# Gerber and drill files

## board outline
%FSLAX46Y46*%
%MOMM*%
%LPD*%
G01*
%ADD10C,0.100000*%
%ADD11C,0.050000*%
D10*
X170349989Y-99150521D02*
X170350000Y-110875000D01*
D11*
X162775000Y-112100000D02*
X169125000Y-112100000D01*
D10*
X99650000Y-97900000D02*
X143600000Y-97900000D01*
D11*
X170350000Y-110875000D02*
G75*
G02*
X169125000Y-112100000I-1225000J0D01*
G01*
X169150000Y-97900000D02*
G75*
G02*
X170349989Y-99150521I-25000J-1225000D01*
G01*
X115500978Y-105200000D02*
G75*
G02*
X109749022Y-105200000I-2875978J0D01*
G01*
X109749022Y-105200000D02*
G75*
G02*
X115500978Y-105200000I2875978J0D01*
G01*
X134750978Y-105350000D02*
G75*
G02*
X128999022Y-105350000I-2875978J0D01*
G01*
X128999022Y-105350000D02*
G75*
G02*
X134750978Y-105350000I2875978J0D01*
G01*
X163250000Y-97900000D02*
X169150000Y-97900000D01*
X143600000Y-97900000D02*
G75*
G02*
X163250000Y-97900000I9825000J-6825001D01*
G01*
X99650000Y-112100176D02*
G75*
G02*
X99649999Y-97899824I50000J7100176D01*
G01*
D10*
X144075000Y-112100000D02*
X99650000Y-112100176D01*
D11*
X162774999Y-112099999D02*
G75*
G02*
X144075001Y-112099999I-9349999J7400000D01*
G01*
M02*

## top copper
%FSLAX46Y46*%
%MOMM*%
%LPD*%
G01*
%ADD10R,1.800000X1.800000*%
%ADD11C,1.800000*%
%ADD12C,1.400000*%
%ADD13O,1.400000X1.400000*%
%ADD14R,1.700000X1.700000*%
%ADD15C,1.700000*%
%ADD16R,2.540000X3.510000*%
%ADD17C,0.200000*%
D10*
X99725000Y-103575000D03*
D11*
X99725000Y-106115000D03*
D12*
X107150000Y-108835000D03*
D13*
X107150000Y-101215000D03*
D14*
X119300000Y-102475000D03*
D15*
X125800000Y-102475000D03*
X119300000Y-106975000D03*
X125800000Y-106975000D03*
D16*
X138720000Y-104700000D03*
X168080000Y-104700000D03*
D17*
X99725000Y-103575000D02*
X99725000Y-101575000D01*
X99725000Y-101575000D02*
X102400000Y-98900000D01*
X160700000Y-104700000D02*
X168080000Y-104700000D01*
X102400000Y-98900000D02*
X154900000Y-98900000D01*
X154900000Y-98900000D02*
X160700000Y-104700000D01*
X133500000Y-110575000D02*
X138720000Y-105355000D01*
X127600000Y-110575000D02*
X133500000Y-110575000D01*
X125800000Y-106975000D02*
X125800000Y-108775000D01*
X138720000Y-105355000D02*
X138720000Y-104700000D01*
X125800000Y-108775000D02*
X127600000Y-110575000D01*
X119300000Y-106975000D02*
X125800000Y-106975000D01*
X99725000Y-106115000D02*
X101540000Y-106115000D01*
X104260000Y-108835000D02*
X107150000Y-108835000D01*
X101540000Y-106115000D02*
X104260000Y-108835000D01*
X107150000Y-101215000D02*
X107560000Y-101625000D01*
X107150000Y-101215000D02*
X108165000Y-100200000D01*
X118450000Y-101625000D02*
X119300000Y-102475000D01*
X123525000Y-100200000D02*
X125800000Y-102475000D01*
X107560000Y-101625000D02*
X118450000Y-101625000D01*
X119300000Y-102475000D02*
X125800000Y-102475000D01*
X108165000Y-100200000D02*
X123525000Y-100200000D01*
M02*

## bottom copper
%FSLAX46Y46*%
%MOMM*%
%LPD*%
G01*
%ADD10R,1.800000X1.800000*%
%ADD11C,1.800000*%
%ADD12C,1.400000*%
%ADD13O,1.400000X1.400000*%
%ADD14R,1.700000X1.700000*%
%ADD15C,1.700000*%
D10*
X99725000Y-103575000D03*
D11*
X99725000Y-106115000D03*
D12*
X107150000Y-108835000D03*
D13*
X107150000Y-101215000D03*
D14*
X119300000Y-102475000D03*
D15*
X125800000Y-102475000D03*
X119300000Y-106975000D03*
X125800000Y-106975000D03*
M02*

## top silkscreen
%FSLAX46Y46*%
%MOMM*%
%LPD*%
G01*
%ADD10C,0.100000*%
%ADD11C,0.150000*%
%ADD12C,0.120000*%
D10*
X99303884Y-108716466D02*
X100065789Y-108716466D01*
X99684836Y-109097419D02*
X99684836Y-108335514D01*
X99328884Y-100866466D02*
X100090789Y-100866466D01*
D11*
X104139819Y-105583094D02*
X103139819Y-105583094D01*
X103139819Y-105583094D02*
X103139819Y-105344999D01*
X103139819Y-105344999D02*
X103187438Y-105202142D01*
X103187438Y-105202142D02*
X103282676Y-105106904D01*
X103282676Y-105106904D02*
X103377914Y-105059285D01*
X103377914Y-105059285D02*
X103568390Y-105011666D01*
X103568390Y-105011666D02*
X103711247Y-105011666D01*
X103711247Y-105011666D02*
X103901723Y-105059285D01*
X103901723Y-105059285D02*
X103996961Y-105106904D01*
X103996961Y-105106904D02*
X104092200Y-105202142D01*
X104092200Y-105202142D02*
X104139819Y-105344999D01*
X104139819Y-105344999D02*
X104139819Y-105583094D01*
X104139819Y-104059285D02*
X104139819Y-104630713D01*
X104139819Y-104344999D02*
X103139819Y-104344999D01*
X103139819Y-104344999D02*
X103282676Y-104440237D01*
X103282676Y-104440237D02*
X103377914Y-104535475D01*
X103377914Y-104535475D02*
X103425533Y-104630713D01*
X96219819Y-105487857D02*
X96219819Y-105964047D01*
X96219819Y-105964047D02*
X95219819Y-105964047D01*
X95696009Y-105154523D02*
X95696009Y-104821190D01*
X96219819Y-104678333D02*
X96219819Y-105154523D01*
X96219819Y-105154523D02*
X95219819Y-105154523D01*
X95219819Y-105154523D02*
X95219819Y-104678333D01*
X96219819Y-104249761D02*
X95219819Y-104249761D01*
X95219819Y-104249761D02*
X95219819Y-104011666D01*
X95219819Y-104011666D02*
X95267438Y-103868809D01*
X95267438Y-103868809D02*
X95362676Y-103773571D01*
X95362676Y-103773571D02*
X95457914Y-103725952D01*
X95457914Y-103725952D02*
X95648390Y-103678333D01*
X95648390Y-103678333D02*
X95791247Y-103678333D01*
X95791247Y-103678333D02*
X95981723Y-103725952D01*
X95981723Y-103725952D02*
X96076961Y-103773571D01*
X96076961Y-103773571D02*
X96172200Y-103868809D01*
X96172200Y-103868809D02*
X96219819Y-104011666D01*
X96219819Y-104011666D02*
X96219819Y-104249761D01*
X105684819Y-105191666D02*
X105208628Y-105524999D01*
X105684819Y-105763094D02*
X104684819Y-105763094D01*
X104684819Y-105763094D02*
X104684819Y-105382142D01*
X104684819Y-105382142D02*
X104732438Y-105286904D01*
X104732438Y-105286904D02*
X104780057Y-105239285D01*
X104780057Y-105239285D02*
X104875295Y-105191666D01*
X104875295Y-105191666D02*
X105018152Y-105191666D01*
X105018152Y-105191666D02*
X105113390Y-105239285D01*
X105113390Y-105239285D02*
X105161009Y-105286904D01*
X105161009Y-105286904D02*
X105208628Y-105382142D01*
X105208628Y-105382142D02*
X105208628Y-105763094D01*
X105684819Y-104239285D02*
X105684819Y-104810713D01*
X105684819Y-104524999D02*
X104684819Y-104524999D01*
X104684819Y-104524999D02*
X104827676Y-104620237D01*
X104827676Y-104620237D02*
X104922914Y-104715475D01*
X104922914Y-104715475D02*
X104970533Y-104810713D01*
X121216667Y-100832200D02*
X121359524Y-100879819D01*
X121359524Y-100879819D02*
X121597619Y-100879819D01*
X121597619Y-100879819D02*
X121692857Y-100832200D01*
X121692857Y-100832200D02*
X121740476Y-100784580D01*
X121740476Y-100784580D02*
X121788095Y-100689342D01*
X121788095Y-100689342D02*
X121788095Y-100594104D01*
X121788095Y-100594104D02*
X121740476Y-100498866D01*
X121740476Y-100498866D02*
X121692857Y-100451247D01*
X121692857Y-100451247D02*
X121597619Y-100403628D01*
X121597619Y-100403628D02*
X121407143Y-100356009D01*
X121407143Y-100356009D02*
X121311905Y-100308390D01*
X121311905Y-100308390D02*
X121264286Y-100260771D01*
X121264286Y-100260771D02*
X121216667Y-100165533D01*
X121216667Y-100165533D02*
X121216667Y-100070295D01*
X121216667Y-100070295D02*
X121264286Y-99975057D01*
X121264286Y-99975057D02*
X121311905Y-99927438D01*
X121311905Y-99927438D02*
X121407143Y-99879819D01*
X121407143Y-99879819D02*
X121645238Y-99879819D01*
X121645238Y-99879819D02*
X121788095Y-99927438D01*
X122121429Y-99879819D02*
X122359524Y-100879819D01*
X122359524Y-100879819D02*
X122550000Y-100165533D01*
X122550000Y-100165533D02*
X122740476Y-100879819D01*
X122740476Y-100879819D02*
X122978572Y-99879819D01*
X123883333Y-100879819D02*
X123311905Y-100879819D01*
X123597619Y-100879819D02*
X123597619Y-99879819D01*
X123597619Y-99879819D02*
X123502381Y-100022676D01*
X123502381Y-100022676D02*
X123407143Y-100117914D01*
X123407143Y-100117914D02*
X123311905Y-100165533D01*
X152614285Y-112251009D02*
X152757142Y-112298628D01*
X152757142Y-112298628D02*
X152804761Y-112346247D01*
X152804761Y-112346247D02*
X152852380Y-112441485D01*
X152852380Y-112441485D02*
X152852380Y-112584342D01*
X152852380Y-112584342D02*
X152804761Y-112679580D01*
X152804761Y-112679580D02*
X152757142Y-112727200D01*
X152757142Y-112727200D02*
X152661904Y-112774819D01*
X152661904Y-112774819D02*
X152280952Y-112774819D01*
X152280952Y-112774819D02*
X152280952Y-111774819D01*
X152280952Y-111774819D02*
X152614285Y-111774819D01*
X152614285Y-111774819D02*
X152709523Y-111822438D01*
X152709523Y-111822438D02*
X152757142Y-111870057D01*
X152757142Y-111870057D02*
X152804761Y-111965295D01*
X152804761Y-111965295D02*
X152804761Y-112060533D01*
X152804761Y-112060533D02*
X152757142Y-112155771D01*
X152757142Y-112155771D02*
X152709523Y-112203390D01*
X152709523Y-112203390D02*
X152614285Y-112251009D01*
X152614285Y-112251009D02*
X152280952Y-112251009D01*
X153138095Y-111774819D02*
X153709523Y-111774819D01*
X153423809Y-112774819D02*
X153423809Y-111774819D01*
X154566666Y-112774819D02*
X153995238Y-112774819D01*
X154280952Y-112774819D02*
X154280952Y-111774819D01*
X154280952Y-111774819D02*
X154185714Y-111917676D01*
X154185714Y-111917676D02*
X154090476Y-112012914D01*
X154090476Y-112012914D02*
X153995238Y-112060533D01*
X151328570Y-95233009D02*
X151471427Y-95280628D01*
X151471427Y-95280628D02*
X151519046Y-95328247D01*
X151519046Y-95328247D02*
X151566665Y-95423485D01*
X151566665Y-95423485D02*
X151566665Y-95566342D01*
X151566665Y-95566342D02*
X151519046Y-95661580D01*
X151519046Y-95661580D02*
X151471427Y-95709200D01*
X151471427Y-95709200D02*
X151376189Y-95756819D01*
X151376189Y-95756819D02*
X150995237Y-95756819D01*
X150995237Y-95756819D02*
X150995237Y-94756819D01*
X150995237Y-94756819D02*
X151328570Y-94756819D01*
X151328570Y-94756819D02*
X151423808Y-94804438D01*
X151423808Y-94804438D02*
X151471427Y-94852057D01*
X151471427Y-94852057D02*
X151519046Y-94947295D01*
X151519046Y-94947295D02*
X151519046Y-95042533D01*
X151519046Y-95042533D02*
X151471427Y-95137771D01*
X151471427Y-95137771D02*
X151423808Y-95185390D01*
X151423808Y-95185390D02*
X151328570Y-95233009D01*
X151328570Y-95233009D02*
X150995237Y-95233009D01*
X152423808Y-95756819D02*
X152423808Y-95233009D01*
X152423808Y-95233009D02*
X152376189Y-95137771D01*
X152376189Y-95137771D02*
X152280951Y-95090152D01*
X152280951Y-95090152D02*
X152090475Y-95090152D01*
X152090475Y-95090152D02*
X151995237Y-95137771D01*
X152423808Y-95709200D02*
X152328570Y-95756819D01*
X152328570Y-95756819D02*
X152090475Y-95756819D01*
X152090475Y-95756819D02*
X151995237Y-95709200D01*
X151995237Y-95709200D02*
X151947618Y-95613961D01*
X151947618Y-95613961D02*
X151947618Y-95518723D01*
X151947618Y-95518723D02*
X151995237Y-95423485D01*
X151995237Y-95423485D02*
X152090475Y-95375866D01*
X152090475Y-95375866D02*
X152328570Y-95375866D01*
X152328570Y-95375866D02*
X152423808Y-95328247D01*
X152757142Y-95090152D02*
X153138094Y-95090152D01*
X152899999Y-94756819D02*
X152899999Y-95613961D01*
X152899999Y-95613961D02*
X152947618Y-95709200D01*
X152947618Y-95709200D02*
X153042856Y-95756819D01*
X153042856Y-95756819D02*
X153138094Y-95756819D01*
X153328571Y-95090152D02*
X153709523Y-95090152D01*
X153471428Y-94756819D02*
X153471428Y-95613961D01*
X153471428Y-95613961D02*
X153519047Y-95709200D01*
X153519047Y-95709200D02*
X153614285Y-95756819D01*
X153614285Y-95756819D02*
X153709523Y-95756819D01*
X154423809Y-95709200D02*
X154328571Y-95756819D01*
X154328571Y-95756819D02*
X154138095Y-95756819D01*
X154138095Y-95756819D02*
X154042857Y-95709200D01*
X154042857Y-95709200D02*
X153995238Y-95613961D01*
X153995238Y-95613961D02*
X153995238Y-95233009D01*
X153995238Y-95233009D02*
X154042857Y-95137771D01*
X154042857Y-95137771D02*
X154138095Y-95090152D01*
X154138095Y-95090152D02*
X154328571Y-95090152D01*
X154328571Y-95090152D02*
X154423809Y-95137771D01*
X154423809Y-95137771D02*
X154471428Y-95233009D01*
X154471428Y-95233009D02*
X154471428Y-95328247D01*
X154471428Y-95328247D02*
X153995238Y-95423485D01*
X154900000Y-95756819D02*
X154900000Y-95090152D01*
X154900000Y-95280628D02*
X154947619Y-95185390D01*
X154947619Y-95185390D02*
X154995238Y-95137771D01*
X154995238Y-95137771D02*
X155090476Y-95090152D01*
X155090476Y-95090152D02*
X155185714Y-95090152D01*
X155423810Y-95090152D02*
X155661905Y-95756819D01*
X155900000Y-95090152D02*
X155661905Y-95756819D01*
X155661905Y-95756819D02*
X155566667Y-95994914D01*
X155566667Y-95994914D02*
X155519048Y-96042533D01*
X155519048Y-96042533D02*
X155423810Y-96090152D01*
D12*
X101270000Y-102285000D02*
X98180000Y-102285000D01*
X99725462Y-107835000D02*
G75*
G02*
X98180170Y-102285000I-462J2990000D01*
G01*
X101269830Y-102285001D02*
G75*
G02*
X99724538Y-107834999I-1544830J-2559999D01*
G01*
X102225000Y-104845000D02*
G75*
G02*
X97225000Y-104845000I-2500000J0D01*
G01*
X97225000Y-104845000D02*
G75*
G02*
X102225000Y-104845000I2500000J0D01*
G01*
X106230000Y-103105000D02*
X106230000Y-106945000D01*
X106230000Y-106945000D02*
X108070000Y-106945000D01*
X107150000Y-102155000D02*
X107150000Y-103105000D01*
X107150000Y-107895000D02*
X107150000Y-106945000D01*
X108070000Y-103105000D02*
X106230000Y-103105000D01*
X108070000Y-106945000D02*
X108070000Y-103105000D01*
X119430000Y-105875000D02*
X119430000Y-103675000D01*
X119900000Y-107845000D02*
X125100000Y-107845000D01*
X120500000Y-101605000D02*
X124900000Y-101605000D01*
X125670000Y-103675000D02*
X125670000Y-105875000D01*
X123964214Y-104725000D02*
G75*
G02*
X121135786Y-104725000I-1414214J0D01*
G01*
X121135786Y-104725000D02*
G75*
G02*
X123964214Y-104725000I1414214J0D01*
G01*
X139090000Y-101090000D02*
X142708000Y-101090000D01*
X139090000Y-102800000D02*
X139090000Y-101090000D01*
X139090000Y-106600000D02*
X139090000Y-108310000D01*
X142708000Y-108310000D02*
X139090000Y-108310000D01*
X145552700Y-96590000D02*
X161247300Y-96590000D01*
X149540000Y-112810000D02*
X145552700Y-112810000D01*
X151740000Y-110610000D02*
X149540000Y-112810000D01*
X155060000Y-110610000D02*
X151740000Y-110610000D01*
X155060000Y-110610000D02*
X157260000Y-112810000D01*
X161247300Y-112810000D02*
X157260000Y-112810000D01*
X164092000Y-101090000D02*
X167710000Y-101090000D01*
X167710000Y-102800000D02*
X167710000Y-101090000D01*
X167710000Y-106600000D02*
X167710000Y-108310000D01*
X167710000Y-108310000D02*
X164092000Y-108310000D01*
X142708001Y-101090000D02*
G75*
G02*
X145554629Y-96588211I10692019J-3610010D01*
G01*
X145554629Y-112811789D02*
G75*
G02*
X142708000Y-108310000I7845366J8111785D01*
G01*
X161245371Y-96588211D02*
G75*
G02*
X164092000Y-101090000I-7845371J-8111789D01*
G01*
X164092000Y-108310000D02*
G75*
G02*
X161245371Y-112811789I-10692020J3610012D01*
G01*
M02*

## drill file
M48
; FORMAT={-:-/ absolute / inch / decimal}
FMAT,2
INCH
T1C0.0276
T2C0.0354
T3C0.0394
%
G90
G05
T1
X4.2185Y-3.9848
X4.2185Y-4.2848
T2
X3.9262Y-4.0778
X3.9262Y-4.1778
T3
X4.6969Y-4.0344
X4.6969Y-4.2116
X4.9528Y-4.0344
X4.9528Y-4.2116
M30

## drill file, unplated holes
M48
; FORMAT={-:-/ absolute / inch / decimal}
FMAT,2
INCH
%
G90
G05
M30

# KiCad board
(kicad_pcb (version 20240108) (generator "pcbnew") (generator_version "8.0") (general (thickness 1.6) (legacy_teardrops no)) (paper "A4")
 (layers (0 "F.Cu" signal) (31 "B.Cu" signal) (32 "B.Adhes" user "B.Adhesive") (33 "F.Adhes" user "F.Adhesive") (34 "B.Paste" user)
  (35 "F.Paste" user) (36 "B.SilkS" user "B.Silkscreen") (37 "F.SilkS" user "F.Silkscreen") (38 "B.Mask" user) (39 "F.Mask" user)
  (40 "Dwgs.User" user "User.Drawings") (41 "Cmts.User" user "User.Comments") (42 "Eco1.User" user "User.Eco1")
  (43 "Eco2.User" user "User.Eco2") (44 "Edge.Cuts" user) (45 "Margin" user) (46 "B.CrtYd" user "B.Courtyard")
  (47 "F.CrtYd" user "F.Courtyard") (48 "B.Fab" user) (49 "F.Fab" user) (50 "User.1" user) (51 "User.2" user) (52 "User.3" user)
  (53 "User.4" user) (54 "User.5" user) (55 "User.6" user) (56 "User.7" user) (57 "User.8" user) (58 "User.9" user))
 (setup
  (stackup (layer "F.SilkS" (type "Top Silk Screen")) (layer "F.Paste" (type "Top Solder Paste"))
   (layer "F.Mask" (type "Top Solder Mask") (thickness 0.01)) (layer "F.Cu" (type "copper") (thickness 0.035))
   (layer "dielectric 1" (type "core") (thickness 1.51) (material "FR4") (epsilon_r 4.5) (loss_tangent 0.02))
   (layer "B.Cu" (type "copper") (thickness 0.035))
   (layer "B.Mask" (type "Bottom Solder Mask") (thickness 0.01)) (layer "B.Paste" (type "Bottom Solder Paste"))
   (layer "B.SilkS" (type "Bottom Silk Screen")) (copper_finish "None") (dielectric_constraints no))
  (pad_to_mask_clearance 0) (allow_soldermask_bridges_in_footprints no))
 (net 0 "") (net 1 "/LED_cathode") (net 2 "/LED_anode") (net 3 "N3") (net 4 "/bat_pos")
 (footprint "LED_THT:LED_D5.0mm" (layer "F.Cu") (at 99.725 103.575 -90)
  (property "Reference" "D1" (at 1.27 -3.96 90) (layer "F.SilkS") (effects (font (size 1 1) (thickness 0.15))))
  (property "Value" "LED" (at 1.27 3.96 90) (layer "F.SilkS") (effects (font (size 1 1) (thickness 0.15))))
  (fp_line (start -1.29 -1.545) (end -1.29 1.545) (stroke (width 0.12) (type solid)) (layer "F.SilkS"))
  (fp_arc (start 4.26 -0.000462) (mid 2.072002 2.880433) (end -1.29 1.54483) (stroke (width 0.12) (type solid)) (layer "F.SilkS"))
  (fp_arc (start -1.29 -1.54483) (mid 2.072002 -2.880433) (end 4.26 0.000462) (stroke (width 0.12) (type solid)) (layer "F.SilkS"))
  (fp_circle (center 1.27 0) (end 3.77 0) (stroke (width 0.12) (type solid)) (fill none) (layer "F.SilkS"))
  (pad "1" thru_hole rect (at 0 0 270) (size 1.8 1.8) (drill 0.9) (layers "*.Cu" "*.Mask") (remove_unused_layers no) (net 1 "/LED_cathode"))
  (pad "2" thru_hole circle (at 2.54 0 270) (size 1.8 1.8) (drill 0.9) (layers "*.Cu" "*.Mask") (remove_unused_layers no)
   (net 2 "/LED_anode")))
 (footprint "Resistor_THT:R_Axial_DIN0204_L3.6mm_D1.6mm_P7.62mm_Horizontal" (layer "F.Cu") (at 107.15 108.835 90)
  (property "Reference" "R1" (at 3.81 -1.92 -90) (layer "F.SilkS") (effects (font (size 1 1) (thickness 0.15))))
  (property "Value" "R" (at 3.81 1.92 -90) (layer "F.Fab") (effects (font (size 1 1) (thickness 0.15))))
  (fp_line (start 5.73 -0.92) (end 1.89 -0.92) (stroke (width 0.12) (type solid)) (layer "F.SilkS"))
  (fp_line (start 1.89 -0.92) (end 1.89 0.92) (stroke (width 0.12) (type solid)) (layer "F.SilkS"))
  (fp_line (start 6.68 0) (end 5.73 0) (stroke (width 0.12) (type solid)) (layer "F.SilkS"))
  (fp_line (start 0.94 0) (end 1.89 0) (stroke (width 0.12) (type solid)) (layer "F.SilkS"))
  (fp_line (start 5.73 0.92) (end 5.73 -0.92) (stroke (width 0.12) (type solid)) (layer "F.SilkS"))
  (fp_line (start 1.89 0.92) (end 5.73 0.92) (stroke (width 0.12) (type solid)) (layer "F.SilkS"))
  (pad "1" thru_hole circle (at 0 0 90) (size 1.4 1.4) (drill 0.7) (layers "*.Cu" "*.Mask") (remove_unused_layers no) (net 2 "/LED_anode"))
  (pad "2" thru_hole oval (at 7.62 0 90) (size 1.4 1.4) (drill 0.7) (layers "*.Cu" "*.Mask") (remove_unused_layers no) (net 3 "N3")))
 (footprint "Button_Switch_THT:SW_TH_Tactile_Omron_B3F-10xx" (layer "F.Cu") (at 119.3 102.475)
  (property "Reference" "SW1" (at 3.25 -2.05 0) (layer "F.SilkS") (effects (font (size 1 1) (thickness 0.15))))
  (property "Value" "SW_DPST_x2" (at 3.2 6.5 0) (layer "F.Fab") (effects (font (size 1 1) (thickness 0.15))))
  (fp_line (start 0.13 3.4) (end 0.13 1.2) (stroke (width 0.12) (type solid)) (layer "F.SilkS"))
  (fp_line (start 0.6 5.37) (end 5.8 5.37) (stroke (width 0.12) (type solid)) (layer "F.SilkS"))
  (fp_line (start 1.2 -0.87) (end 5.6 -0.87) (stroke (width 0.12) (type solid)) (layer "F.SilkS"))
  (fp_line (start 6.37 1.2) (end 6.37 3.4) (stroke (width 0.12) (type solid)) (layer "F.SilkS"))
  (fp_circle (center 3.25 2.25) (end 4.25 3.25) (stroke (width 0.12) (type solid)) (fill none) (layer "F.SilkS"))
  (pad "1" thru_hole rect (at 0 0) (size 1.7 1.7) (drill 1) (layers "*.Cu" "*.Mask") (remove_unused_layers no) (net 3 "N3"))
  (pad "1" thru_hole circle (at 6.5 0) (size 1.7 1.7) (drill 1) (layers "*.Cu" "*.Mask") (remove_unused_layers no) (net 3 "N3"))
  (pad "2" thru_hole circle (at 0 4.5) (size 1.7 1.7) (drill 1) (layers "*.Cu" "*.Mask") (remove_unused_layers no) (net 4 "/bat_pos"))
  (pad "2" thru_hole circle (at 6.5 4.5) (size 1.7 1.7) (drill 1) (layers "*.Cu" "*.Mask") (remove_unused_layers no) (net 4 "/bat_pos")))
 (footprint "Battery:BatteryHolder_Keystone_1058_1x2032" (layer "F.Cu") (at 153.4 104.7)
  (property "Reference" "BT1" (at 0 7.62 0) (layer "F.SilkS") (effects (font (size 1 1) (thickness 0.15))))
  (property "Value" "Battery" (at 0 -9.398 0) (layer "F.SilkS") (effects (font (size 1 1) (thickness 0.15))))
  (fp_line (start -14.31 -3.61) (end -10.692 -3.61) (stroke (width 0.12) (type solid)) (layer "F.SilkS"))
  (fp_line (start -14.31 -1.9) (end -14.31 -3.61) (stroke (width 0.12) (type solid)) (layer "F.SilkS"))
  (fp_line (start -14.31 1.9) (end -14.31 3.61) (stroke (width 0.12) (type solid)) (layer "F.SilkS"))
  (fp_line (start -10.692 3.61) (end -14.31 3.61) (stroke (width 0.12) (type solid)) (layer "F.SilkS"))
  (fp_line (start -7.8473 -8.11) (end 7.8473 -8.11) (stroke (width 0.12) (type solid)) (layer "F.SilkS"))
  (fp_line (start -3.86 8.11) (end -7.8473 8.11) (stroke (width 0.12) (type solid)) (layer "F.SilkS"))
  (fp_line (start -1.66 5.91) (end -3.86 8.11) (stroke (width 0.12) (type solid)) (layer "F.SilkS"))
  (fp_line (start 1.66 5.91) (end -1.66 5.91) (stroke (width 0.12) (type solid)) (layer "F.SilkS"))
  (fp_line (start 1.66 5.91) (end 3.86 8.11) (stroke (width 0.12) (type solid)) (layer "F.SilkS"))
  (fp_line (start 7.8473 8.11) (end 3.86 8.11) (stroke (width 0.12) (type solid)) (layer "F.SilkS"))
  (fp_line (start 10.692 -3.61) (end 14.31 -3.61) (stroke (width 0.12) (type solid)) (layer "F.SilkS"))
  (fp_line (start 14.31 -1.9) (end 14.31 -3.61) (stroke (width 0.12) (type solid)) (layer "F.SilkS"))
  (fp_line (start 14.31 1.9) (end 14.31 3.61) (stroke (width 0.12) (type solid)) (layer "F.SilkS"))
  (fp_line (start 14.31 3.61) (end 10.692 3.61) (stroke (width 0.12) (type solid)) (layer "F.SilkS"))
  (fp_arc (start -10.692 -3.61) (mid -9.538084 -6.031244) (end -7.845371 -8.111789) (stroke (width 0.12) (type solid)) (layer "F.SilkS"))
  (fp_arc (start -7.845371 8.111789) (mid -9.538085 6.031244) (end -10.692 3.61) (stroke (width 0.12) (type solid)) (layer "F.SilkS"))
  (fp_arc (start 7.845371 -8.111789) (mid 9.538085 -6.031244) (end 10.692 -3.61) (stroke (width 0.12) (type solid)) (layer "F.SilkS"))
  (fp_arc (start 10.692 3.61) (mid 9.538084 6.031244) (end 7.845371 8.111789) (stroke (width 0.12) (type solid)) (layer "F.SilkS"))
  (pad "1" smd rect (at -14.68 0) (size 2.54 3.51) (layers "F.Cu" "F.Paste" "F.Mask") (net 4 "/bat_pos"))
  (pad "2" smd rect (at 14.68 0) (size 2.54 3.51) (layers "F.Cu" "F.Paste" "F.Mask") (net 1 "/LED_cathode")))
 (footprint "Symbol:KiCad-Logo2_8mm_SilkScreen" (layer "B.Cu") (at 153.6 104.075 180)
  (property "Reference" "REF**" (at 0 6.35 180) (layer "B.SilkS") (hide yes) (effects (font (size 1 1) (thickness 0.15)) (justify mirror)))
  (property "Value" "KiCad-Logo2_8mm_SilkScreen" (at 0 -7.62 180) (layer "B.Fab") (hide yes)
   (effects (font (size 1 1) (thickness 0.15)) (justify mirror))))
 (gr_line (start 170.349989 99.150521) (end 170.35 110.875) (stroke (width 0.1) (type default)) (layer "Edge.Cuts"))
 (gr_line (start 162.775 112.1) (end 169.125 112.1) (stroke (width 0.05) (type default)) (layer "Edge.Cuts"))
 (gr_line (start 99.65 97.9) (end 143.6 97.9) (stroke (width 0.1) (type default)) (layer "Edge.Cuts"))
 (gr_arc (start 170.35 110.875) (mid 169.991206 111.741206) (end 169.125 112.1) (stroke (width 0.05) (type default)) (layer "Edge.Cuts"))
 (gr_arc (start 169.15 97.9) (mid 170.009064 98.27666) (end 170.349989 99.150521) (stroke (width 0.05) (type default)) (layer "Edge.Cuts"))
 (gr_circle (center 112.625 105.2) (end 109.75 105.275) (stroke (width 0.05) (type default)) (fill none) (layer "Edge.Cuts"))
 (gr_circle (center 131.875 105.35) (end 129 105.425) (stroke (width 0.05) (type default)) (fill none) (layer "Edge.Cuts"))
 (gr_line (start 163.25 97.9) (end 169.15 97.9) (stroke (width 0.05) (type default)) (layer "Edge.Cuts"))
 (gr_arc (start 143.6 97.9) (mid 153.425 92.762089) (end 163.25 97.9) (stroke (width 0.05) (type default)) (layer "Edge.Cuts"))
 (gr_arc (start 99.65 112.100176) (mid 92.599648 105) (end 99.649999 97.899824) (stroke (width 0.05) (type default)) (layer "Edge.Cuts"))
 (gr_line (start 144.075 112.1) (end 99.65 112.100176) (stroke (width 0.1) (type default)) (layer "Edge.Cuts"))
 (gr_arc (start 162.775 112.1) (mid 153.425 116.62403) (end 144.075 112.1) (stroke (width 0.05) (type default)) (layer "Edge.Cuts"))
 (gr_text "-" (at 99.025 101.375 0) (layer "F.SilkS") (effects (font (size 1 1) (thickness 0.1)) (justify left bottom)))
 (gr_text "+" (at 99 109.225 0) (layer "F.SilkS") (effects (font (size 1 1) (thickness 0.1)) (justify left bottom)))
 (segment (start 99.725 103.575) (end 99.725 101.575) (width 0.2) (layer "F.Cu") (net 1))
 (segment (start 99.725 101.575) (end 102.4 98.9) (width 0.2) (layer "F.Cu") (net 1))
 (segment (start 160.7 104.7) (end 168.08 104.7) (width 0.2) (layer "F.Cu") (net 1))
 (segment (start 102.4 98.9) (end 154.9 98.9) (width 0.2) (layer "F.Cu") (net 1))
 (segment (start 154.9 98.9) (end 160.7 104.7) (width 0.2) (layer "F.Cu") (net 1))
 (segment (start 133.5 110.575) (end 138.72 105.355) (width 0.2) (layer "F.Cu") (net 4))
 (segment (start 127.6 110.575) (end 133.5 110.575) (width 0.2) (layer "F.Cu") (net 4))
 (segment (start 125.8 106.975) (end 125.8 108.775) (width 0.2) (layer "F.Cu") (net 4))
 (segment (start 138.72 105.355) (end 138.72 104.7) (width 0.2) (layer "F.Cu") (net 4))
 (segment (start 125.8 108.775) (end 127.6 110.575) (width 0.2) (layer "F.Cu") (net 4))
 (segment (start 119.3 106.975) (end 125.8 106.975) (width 0.2) (layer "F.Cu") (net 4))
 (segment (start 99.725 106.115) (end 101.54 106.115) (width 0.2) (layer "F.Cu") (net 2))
 (segment (start 104.26 108.835) (end 107.15 108.835) (width 0.2) (layer "F.Cu") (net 2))
 (segment (start 101.54 106.115) (end 104.26 108.835) (width 0.2) (layer "F.Cu") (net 2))
 (segment (start 107.15 101.215) (end 107.56 101.625) (width 0.2) (layer "F.Cu") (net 3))
 (segment (start 107.15 101.215) (end 108.165 100.2) (width 0.2) (layer "F.Cu") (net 3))
 (segment (start 118.45 101.625) (end 119.3 102.475) (width 0.2) (layer "F.Cu") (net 3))
 (segment (start 123.525 100.2) (end 125.8 102.475) (width 0.2) (layer "F.Cu") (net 3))
 (segment (start 107.56 101.625) (end 118.45 101.625) (width 0.2) (layer "F.Cu") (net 3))
 (segment (start 119.3 102.475) (end 125.8 102.475) (width 0.2) (layer "F.Cu") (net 3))
 (segment (start 108.165 100.2) (end 123.525 100.2) (width 0.2) (layer "F.Cu") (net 3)))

